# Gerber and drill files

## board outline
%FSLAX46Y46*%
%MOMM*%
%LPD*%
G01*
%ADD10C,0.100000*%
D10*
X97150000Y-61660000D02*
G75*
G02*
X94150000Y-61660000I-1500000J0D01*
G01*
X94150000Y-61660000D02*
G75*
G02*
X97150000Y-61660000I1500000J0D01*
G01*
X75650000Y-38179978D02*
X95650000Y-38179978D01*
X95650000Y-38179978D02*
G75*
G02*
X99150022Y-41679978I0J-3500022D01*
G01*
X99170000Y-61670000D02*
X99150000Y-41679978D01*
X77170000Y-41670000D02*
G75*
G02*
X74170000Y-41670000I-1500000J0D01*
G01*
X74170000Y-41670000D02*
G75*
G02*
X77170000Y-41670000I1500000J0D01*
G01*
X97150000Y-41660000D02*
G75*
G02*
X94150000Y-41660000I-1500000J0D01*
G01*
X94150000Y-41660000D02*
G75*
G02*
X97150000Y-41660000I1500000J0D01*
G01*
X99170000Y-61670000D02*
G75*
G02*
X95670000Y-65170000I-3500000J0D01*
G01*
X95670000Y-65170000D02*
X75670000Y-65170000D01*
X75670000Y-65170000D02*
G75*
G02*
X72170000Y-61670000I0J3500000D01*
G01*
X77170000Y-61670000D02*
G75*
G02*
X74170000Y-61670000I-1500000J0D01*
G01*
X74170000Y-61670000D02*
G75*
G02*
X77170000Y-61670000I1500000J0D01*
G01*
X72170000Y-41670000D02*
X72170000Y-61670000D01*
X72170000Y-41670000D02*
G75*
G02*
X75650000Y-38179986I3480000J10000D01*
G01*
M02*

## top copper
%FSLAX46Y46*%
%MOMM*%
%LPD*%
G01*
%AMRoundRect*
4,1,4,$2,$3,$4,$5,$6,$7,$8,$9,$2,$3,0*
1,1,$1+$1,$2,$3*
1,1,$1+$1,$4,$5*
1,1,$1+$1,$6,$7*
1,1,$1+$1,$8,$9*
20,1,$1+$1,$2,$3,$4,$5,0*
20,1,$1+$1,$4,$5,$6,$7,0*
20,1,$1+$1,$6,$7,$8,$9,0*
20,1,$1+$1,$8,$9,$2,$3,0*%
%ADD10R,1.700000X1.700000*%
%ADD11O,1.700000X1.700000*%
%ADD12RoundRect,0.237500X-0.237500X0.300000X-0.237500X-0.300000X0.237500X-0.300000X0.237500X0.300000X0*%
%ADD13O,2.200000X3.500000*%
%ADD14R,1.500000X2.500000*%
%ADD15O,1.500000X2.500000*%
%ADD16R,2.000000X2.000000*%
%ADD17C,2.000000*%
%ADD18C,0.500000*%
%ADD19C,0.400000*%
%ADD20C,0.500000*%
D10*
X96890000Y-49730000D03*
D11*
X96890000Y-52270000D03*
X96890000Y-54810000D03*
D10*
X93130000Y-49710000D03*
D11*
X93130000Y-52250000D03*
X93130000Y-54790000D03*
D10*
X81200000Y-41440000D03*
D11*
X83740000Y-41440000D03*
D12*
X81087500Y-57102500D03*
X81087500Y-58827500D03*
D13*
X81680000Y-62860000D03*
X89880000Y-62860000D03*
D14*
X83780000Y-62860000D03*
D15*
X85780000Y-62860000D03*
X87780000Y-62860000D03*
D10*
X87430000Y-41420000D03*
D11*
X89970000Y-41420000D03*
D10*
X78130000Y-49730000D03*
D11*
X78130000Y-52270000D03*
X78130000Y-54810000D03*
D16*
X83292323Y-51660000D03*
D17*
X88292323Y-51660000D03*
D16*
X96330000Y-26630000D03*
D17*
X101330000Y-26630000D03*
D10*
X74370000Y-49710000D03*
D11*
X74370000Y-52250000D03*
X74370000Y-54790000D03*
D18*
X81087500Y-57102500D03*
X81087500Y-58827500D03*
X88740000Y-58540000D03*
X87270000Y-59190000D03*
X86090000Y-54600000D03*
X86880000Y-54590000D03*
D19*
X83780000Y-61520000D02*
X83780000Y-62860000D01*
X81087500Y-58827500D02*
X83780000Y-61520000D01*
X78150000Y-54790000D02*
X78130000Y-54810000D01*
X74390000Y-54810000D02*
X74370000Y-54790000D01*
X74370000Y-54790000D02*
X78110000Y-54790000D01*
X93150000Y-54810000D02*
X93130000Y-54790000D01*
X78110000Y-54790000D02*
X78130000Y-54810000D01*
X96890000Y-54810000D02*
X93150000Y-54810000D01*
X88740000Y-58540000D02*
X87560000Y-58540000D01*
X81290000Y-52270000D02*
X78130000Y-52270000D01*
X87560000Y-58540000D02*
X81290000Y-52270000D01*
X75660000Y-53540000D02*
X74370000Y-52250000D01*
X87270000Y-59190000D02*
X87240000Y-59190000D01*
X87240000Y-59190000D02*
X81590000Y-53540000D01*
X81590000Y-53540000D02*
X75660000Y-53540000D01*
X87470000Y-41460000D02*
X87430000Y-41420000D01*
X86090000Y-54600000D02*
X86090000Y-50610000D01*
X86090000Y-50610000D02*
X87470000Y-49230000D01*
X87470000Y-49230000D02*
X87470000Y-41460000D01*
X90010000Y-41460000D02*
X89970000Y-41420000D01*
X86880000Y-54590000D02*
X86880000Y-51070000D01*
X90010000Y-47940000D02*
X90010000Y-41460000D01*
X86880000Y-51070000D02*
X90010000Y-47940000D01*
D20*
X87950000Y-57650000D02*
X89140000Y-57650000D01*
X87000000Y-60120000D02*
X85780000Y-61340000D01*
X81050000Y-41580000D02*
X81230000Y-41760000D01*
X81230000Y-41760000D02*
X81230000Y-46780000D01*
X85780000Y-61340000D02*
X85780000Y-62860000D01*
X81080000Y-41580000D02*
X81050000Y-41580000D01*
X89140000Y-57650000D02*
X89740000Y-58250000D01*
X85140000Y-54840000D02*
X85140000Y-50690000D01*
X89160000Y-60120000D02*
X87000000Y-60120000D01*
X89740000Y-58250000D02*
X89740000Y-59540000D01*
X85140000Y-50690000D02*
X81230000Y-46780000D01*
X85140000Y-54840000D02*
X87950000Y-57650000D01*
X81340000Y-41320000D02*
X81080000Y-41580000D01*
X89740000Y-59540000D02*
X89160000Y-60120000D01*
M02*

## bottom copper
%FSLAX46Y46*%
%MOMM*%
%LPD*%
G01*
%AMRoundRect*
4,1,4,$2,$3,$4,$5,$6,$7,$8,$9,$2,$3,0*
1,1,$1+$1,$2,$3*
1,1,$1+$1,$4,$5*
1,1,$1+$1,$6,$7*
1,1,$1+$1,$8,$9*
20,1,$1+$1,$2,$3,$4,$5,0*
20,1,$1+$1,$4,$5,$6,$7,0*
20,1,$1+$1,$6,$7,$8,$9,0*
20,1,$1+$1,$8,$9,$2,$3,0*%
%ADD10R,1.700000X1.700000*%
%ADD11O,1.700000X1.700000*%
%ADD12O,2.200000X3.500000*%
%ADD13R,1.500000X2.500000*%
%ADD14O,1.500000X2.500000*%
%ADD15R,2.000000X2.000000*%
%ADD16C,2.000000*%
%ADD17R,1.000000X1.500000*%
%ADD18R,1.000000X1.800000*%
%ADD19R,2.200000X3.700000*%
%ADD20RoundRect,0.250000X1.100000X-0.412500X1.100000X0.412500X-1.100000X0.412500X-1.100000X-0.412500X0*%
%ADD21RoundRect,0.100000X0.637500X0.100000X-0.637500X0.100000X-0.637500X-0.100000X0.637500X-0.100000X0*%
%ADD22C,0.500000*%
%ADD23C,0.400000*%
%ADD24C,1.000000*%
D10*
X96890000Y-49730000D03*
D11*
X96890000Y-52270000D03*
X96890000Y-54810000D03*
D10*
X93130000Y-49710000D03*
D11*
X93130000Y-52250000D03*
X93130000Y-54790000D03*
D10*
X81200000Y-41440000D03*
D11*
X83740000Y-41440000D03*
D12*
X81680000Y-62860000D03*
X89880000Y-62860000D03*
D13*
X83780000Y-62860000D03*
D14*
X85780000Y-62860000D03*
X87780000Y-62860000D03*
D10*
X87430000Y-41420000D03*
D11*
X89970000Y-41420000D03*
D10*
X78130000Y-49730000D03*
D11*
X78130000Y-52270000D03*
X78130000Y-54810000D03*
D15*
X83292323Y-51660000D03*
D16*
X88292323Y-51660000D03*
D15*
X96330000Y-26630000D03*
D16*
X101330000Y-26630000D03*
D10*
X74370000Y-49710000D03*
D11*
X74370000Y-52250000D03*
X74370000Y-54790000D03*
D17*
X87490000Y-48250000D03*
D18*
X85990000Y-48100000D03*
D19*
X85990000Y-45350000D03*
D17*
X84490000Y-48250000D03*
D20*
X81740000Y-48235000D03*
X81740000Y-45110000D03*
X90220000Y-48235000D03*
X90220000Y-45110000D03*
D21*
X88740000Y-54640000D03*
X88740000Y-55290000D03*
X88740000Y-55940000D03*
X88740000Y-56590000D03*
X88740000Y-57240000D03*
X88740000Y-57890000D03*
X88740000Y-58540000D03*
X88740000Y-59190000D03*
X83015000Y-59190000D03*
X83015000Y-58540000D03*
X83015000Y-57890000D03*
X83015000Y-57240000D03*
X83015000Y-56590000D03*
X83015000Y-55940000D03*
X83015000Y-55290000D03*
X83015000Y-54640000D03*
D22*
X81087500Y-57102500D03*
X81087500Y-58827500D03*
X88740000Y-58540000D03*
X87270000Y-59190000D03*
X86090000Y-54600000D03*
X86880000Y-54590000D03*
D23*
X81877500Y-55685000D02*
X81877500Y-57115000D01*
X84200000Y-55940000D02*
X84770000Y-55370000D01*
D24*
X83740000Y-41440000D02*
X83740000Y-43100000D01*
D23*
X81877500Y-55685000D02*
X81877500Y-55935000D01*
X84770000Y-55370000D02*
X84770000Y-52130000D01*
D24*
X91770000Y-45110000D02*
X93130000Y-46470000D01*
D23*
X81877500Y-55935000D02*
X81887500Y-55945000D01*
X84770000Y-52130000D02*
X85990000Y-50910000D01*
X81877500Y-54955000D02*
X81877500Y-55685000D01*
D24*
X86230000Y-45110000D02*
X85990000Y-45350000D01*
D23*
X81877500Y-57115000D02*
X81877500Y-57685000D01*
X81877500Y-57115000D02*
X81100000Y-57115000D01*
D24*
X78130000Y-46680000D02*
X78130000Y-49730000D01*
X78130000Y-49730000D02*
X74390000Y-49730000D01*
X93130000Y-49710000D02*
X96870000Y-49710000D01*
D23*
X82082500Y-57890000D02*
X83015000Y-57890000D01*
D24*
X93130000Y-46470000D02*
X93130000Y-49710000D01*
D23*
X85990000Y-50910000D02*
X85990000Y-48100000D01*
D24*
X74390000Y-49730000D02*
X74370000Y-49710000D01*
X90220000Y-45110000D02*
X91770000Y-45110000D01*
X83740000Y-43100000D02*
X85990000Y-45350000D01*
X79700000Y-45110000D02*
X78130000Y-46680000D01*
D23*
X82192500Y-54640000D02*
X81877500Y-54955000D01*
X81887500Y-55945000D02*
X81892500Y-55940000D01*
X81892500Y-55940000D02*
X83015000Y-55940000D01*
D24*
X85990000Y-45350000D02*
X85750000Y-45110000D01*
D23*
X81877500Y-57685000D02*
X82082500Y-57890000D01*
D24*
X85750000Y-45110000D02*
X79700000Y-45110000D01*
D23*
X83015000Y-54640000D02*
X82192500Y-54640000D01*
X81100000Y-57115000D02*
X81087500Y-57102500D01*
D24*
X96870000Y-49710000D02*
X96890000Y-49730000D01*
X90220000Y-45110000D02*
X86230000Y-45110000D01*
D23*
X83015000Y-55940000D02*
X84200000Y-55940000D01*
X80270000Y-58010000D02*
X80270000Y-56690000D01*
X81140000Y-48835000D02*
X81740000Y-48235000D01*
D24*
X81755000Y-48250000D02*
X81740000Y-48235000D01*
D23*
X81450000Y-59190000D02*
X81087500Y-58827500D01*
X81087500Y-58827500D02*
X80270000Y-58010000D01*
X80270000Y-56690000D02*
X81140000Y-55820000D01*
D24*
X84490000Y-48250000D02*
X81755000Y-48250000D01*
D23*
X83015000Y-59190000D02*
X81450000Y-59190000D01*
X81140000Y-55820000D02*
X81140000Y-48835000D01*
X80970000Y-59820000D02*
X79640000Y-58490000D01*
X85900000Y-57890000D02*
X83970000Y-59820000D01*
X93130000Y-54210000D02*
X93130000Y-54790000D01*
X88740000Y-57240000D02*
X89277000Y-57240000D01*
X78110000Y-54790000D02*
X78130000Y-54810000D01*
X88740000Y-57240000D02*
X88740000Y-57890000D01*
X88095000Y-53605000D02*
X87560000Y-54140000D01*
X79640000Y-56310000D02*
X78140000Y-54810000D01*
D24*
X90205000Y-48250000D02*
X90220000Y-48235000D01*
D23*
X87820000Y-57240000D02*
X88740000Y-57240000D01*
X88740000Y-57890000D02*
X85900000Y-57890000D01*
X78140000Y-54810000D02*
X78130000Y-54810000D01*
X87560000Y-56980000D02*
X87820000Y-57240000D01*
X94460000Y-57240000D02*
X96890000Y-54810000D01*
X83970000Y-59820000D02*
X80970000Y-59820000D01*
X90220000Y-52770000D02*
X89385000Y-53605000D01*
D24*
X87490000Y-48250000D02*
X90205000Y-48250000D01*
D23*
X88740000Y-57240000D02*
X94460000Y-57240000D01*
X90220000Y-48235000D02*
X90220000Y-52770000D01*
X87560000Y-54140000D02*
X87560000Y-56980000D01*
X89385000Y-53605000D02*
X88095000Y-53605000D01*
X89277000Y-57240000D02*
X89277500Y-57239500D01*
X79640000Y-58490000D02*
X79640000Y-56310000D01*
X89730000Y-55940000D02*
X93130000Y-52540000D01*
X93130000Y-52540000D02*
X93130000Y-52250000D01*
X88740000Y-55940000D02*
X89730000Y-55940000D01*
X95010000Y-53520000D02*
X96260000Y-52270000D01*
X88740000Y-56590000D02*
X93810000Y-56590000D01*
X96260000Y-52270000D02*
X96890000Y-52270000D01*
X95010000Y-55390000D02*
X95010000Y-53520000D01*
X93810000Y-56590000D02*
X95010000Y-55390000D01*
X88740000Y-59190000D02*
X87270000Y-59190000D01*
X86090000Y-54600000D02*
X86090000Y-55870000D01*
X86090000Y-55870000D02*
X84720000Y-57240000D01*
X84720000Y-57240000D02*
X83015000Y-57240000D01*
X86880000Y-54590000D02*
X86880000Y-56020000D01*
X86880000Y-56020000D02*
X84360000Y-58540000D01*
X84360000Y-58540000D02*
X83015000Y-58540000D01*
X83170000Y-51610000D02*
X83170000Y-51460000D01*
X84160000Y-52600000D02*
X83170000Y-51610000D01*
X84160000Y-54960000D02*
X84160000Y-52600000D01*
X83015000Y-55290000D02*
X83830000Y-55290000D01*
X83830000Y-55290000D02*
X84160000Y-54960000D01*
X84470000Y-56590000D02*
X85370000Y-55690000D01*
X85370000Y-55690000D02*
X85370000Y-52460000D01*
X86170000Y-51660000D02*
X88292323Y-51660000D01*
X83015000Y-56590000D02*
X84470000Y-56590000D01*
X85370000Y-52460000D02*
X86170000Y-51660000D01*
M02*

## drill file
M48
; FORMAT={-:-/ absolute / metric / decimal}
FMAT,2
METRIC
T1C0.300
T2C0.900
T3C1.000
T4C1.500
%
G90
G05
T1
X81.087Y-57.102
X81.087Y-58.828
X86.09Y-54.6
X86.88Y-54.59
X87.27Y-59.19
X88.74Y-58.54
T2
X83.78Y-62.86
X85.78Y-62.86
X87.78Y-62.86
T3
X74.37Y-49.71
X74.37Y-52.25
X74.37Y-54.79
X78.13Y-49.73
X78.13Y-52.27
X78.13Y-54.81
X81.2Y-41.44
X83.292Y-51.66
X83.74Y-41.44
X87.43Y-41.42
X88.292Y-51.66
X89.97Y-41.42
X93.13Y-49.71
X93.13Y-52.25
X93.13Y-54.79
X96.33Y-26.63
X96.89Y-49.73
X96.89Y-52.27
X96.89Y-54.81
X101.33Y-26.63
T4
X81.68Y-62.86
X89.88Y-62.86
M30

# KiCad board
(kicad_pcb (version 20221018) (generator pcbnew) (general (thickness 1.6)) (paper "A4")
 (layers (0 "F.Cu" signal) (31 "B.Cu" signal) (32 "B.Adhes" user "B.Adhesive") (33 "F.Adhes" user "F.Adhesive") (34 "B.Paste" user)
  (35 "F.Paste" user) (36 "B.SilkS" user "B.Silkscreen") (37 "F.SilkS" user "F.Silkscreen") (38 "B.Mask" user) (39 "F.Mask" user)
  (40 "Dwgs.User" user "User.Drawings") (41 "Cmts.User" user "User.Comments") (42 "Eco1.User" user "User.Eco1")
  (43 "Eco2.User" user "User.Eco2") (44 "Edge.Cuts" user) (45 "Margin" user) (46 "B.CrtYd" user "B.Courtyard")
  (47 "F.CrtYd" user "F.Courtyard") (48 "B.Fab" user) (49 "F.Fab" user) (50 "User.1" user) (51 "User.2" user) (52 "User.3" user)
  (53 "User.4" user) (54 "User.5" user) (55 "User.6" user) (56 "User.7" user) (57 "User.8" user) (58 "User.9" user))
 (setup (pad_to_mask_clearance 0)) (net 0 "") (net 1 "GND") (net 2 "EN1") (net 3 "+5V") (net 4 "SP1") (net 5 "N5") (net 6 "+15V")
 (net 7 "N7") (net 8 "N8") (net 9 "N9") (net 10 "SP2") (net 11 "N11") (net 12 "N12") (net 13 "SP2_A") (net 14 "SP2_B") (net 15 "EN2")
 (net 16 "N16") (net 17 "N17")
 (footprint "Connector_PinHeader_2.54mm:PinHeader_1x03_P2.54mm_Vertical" (layer "F.Cu") (at 96.89 49.73)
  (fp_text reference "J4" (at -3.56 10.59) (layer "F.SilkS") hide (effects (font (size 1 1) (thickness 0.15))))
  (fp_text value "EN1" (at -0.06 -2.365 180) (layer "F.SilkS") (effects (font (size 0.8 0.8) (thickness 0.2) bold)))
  (pad "1" thru_hole rect (at 0 0) (size 1.7 1.7) (drill 1) (layers "*.Cu" "*.Mask") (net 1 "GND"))
  (pad "2" thru_hole oval (at 0 2.54) (size 1.7 1.7) (drill 1) (layers "*.Cu" "*.Mask") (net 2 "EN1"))
  (pad "3" thru_hole oval (at 0 5.08) (size 1.7 1.7) (drill 1) (layers "*.Cu" "*.Mask") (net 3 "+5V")))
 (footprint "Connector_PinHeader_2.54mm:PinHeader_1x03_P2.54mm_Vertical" (layer "F.Cu") (at 93.13 49.71)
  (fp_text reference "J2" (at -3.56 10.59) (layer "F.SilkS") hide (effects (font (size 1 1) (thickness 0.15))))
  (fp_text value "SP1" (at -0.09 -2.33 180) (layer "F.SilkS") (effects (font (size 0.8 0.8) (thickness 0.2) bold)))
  (pad "1" thru_hole rect (at 0 0) (size 1.7 1.7) (drill 1) (layers "*.Cu" "*.Mask") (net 1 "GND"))
  (pad "2" thru_hole oval (at 0 2.54) (size 1.7 1.7) (drill 1) (layers "*.Cu" "*.Mask") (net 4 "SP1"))
  (pad "3" thru_hole oval (at 0 5.08) (size 1.7 1.7) (drill 1) (layers "*.Cu" "*.Mask") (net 3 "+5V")))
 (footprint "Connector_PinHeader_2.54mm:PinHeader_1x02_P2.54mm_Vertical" (layer "F.Cu") (at 81.2 41.44 90)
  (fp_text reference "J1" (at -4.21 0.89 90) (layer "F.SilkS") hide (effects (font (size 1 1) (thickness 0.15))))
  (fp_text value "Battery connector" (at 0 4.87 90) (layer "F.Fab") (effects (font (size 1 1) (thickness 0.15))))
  (pad "1" thru_hole rect (at 0 0 90) (size 1.7 1.7) (drill 1) (layers "*.Cu" "*.Mask") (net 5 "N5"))
  (pad "2" thru_hole oval (at 0 2.54 90) (size 1.7 1.7) (drill 1) (layers "*.Cu" "*.Mask") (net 1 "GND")))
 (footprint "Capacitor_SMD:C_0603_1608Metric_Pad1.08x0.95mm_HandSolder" (layer "F.Cu") (at 81.0875 57.965 -90)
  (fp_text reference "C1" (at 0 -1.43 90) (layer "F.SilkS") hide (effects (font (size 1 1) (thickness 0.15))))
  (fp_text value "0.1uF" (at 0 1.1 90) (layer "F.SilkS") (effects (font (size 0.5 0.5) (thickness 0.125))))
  (pad "1" smd roundrect (at -0.8625 0 270) (size 1.075 0.95) (layers "F.Cu" "F.Paste" "F.Mask") (roundrect_rratio 0.25) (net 1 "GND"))
  (pad "2" smd roundrect (at 0.8625 0 270) (size 1.075 0.95) (layers "F.Cu" "F.Paste" "F.Mask") (roundrect_rratio 0.25) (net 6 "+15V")))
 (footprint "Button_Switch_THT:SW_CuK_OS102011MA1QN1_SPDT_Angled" (layer "F.Cu") (at 83.78 62.86)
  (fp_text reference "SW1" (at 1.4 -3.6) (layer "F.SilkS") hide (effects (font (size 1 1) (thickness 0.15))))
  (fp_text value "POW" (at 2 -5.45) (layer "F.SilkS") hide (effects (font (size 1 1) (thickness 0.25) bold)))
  (pad "" thru_hole oval (at -2.1 0) (size 2.2 3.5) (drill 1.5) (layers "*.Cu" "*.Mask"))
  (pad "" thru_hole oval (at 6.1 0) (size 2.2 3.5) (drill 1.5) (layers "*.Cu" "*.Mask"))
  (pad "1" thru_hole rect (at 0 0) (size 1.5 2.5) (drill 0.9) (layers "*.Cu" "*.Mask") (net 6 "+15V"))
  (pad "2" thru_hole oval (at 2 0) (size 1.5 2.5) (drill 0.9) (layers "*.Cu" "*.Mask") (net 5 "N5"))
  (pad "3" thru_hole oval (at 4 0) (size 1.5 2.5) (drill 0.9) (layers "*.Cu" "*.Mask") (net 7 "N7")))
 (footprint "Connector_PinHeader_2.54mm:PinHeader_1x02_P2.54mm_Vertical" (layer "F.Cu") (at 87.43 41.42 90)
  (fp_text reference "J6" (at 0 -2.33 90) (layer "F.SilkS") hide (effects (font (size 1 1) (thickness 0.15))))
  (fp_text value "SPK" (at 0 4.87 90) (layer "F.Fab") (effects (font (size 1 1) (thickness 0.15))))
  (pad "1" thru_hole rect (at 0 0 90) (size 1.7 1.7) (drill 1) (layers "*.Cu" "*.Mask") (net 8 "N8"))
  (pad "2" thru_hole oval (at 0 2.54 90) (size 1.7 1.7) (drill 1) (layers "*.Cu" "*.Mask") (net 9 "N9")))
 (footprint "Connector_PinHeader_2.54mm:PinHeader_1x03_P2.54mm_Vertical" (layer "F.Cu") (at 78.13 49.73)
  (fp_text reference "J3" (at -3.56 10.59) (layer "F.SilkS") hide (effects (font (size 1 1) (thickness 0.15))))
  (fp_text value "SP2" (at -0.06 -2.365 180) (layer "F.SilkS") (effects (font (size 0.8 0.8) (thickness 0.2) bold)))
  (pad "1" thru_hole rect (at 0 0) (size 1.7 1.7) (drill 1) (layers "*.Cu" "*.Mask") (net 1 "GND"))
  (pad "2" thru_hole oval (at 0 2.54) (size 1.7 1.7) (drill 1) (layers "*.Cu" "*.Mask") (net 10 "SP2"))
  (pad "3" thru_hole oval (at 0 5.08) (size 1.7 1.7) (drill 1) (layers "*.Cu" "*.Mask") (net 3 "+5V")))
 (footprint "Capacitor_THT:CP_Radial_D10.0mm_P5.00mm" (layer "F.Cu") (at 83.292323 51.66)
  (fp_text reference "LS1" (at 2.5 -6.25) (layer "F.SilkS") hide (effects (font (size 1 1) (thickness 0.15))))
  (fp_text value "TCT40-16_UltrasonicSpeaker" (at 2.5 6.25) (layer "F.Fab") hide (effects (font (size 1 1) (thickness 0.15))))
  (pad "1" thru_hole rect (at 0 0) (size 2 2) (drill 1) (layers "*.Cu" "*.Mask") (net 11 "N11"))
  (pad "2" thru_hole circle (at 5 0) (size 2 2) (drill 1) (layers "*.Cu" "*.Mask") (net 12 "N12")))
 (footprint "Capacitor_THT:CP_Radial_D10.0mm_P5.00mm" (layer "F.Cu") (at 96.33 26.63)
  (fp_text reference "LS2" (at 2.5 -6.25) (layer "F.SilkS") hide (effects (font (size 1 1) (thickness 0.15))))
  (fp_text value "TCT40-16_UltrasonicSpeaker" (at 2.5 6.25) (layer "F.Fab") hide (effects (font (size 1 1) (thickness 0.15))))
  (pad "1" thru_hole rect (at 0 0) (size 2 2) (drill 1) (layers "*.Cu" "*.Mask") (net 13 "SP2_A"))
  (pad "2" thru_hole circle (at 5 0) (size 2 2) (drill 1) (layers "*.Cu" "*.Mask") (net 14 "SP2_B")))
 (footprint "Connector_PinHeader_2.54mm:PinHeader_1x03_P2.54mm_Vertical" (layer "F.Cu") (at 74.37 49.71)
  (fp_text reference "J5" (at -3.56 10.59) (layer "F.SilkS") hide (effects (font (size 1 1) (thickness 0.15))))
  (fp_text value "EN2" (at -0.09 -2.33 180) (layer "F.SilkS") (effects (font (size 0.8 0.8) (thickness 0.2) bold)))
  (pad "1" thru_hole rect (at 0 0) (size 1.7 1.7) (drill 1) (layers "*.Cu" "*.Mask") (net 1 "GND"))
  (pad "2" thru_hole oval (at 0 2.54) (size 1.7 1.7) (drill 1) (layers "*.Cu" "*.Mask") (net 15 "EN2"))
  (pad "3" thru_hole oval (at 0 5.08) (size 1.7 1.7) (drill 1) (layers "*.Cu" "*.Mask") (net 3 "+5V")))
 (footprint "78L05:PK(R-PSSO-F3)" (layer "B.Cu") (at 85.99 44.6 180)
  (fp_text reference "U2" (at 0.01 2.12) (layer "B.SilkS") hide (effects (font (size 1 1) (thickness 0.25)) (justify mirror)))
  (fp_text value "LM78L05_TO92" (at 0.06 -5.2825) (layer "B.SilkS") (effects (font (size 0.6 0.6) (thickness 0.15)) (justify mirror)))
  (pad "1" smd rect (at -1.5 -3.65 180) (size 1 1.5) (layers "B.Cu" "B.Paste" "B.Mask") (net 3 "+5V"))
  (pad "2" smd rect (at 0 -3.5 180) (size 1 1.8) (layers "B.Cu" "B.Paste" "B.Mask") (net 1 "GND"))
  (pad "2" smd rect (at 0 -0.75 180) (size 2.2 3.7) (layers "B.Cu" "B.Paste" "B.Mask") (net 1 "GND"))
  (pad "3" smd rect (at 1.5 -3.65 180) (size 1 1.5) (layers "B.Cu" "B.Paste" "B.Mask") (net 6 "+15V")))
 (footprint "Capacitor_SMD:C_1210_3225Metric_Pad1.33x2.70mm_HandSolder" (layer "B.Cu") (at 81.74 46.6725 90)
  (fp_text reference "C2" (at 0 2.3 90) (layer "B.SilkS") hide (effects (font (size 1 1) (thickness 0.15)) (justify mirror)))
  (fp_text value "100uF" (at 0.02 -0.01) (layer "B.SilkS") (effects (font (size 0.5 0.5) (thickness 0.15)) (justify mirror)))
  (pad "1" smd roundrect (at -1.5625 0 90) (size 1.325 2.7) (layers "B.Cu" "B.Paste" "B.Mask") (roundrect_rratio 0.188679) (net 6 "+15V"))
  (pad "2" smd roundrect (at 1.5625 0 90) (size 1.325 2.7) (layers "B.Cu" "B.Paste" "B.Mask") (roundrect_rratio 0.188679) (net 1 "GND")))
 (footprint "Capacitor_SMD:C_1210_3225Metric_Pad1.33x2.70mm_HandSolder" (layer "B.Cu") (at 90.22 46.6725 90)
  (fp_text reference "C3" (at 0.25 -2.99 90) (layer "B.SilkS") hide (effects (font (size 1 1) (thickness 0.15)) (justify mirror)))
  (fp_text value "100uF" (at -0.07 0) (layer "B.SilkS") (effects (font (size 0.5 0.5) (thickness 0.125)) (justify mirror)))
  (pad "1" smd roundrect (at -1.5625 0 90) (size 1.325 2.7) (layers "B.Cu" "B.Paste" "B.Mask") (roundrect_rratio 0.188679) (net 3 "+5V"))
  (pad "2" smd roundrect (at 1.5625 0 90) (size 1.325 2.7) (layers "B.Cu" "B.Paste" "B.Mask") (roundrect_rratio 0.188679) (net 1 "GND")))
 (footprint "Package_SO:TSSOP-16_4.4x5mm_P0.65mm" (layer "B.Cu") (at 85.8775 56.915 180)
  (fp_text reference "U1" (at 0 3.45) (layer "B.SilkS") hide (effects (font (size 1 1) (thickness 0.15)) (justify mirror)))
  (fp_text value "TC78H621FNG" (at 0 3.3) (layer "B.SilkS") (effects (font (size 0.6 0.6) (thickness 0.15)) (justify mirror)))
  (pad "1" smd roundrect (at -2.8625 2.275 180) (size 1.475 0.4) (layers "B.Cu" "B.Paste" "B.Mask") (roundrect_rratio 0.25) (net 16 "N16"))
  (pad "2" smd roundrect (at -2.8625 1.625 180) (size 1.475 0.4) (layers "B.Cu" "B.Paste" "B.Mask") (roundrect_rratio 0.25) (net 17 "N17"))
  (pad "3" smd roundrect (at -2.8625 0.975 180) (size 1.475 0.4) (layers "B.Cu" "B.Paste" "B.Mask") (roundrect_rratio 0.25) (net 4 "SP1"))
  (pad "4" smd roundrect (at -2.8625 0.325 180) (size 1.475 0.4) (layers "B.Cu" "B.Paste" "B.Mask") (roundrect_rratio 0.25) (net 2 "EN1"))
  (pad "5" smd roundrect (at -2.8625 -0.325 180) (size 1.475 0.4) (layers "B.Cu" "B.Paste" "B.Mask") (roundrect_rratio 0.25) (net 3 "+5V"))
  (pad "6" smd roundrect (at -2.8625 -0.975 180) (size 1.475 0.4) (layers "B.Cu" "B.Paste" "B.Mask") (roundrect_rratio 0.25) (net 3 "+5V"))
  (pad "7" smd roundrect (at -2.8625 -1.625 180) (size 1.475 0.4) (layers "B.Cu" "B.Paste" "B.Mask") (roundrect_rratio 0.25) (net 10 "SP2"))
  (pad "8" smd roundrect (at -2.8625 -2.275 180) (size 1.475 0.4) (layers "B.Cu" "B.Paste" "B.Mask") (roundrect_rratio 0.25) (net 15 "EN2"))
  (pad "9" smd roundrect (at 2.8625 -2.275 180) (size 1.475 0.4) (layers "B.Cu" "B.Paste" "B.Mask") (roundrect_rratio 0.25) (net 6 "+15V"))
  (pad "10" smd roundrect (at 2.8625 -1.625 180) (size 1.475 0.4) (layers "B.Cu" "B.Paste" "B.Mask") (roundrect_rratio 0.25) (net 9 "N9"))
  (pad "11" smd roundrect (at 2.8625 -0.975 180) (size 1.475 0.4) (layers "B.Cu" "B.Paste" "B.Mask") (roundrect_rratio 0.25) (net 1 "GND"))
  (pad "12" smd roundrect (at 2.8625 -0.325 180) (size 1.475 0.4) (layers "B.Cu" "B.Paste" "B.Mask") (roundrect_rratio 0.25) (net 8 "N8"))
  (pad "13" smd roundrect (at 2.8625 0.325 180) (size 1.475 0.4) (layers "B.Cu" "B.Paste" "B.Mask") (roundrect_rratio 0.25) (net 12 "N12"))
  (pad "14" smd roundrect (at 2.8625 0.975 180) (size 1.475 0.4) (layers "B.Cu" "B.Paste" "B.Mask") (roundrect_rratio 0.25) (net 1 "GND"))
  (pad "15" smd roundrect (at 2.8625 1.625 180) (size 1.475 0.4) (layers "B.Cu" "B.Paste" "B.Mask") (roundrect_rratio 0.25) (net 11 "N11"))
  (pad "16" smd roundrect (at 2.8625 2.275 180) (size 1.475 0.4) (layers "B.Cu" "B.Paste" "B.Mask") (roundrect_rratio 0.25) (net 1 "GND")))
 (gr_circle (center 95.65 61.66) (end 95.65 60.16) (stroke (width 0.1) (type solid)) (fill none) (layer "Edge.Cuts"))
 (gr_line (start 75.65 38.179978) (end 95.65 38.179978) (stroke (width 0.1) (type default)) (layer "Edge.Cuts"))
 (gr_arc (start 95.65 38.179978) (mid 98.124874 39.205104) (end 99.15 41.679978) (stroke (width 0.1) (type default)) (layer "Edge.Cuts"))
 (gr_line (start 99.17 61.67) (end 99.15 41.679978) (stroke (width 0.1) (type default)) (layer "Edge.Cuts"))
 (gr_circle (center 75.67 41.67) (end 75.67 43.17) (stroke (width 0.1) (type solid)) (fill none) (layer "Edge.Cuts"))
 (gr_circle (center 95.65 41.66) (end 95.65 40.16) (stroke (width 0.1) (type solid)) (fill none) (layer "Edge.Cuts"))
 (gr_arc (start 99.17 61.67) (mid 98.144874 64.144874) (end 95.67 65.17) (stroke (width 0.1) (type default)) (layer "Edge.Cuts"))
 (gr_line (start 95.67 65.17) (end 75.67 65.17) (stroke (width 0.1) (type default)) (layer "Edge.Cuts"))
 (gr_arc (start 75.67 65.17) (mid 73.195126 64.144874) (end 72.17 61.67) (stroke (width 0.1) (type default)) (layer "Edge.Cuts"))
 (gr_circle (center 75.67 61.67) (end 75.67 63.17) (stroke (width 0.1) (type solid)) (fill none) (layer "Edge.Cuts"))
 (gr_line (start 72.17 41.67) (end 72.17 61.67) (stroke (width 0.1) (type default)) (layer "Edge.Cuts"))
 (gr_arc (start 72.17 41.67) (mid 73.185724 39.202792) (end 75.65 38.179978) (stroke (width 0.1) (type default)) (layer "Edge.Cuts"))
 (via (at 81.0875 57.1025) (size 0.5) (drill 0.3) (layers "F.Cu" "B.Cu") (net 1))
 (segment (start 81.8775 55.685) (end 81.8775 57.115) (width 0.4) (layer "B.Cu") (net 1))
 (segment (start 84.2 55.94) (end 84.77 55.37) (width 0.4) (layer "B.Cu") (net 1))
 (segment (start 83.74 41.44) (end 83.74 43.1) (width 1) (layer "B.Cu") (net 1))
 (segment (start 81.8775 55.685) (end 81.8775 55.935) (width 0.4) (layer "B.Cu") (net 1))
 (segment (start 84.77 55.37) (end 84.77 52.13) (width 0.4) (layer "B.Cu") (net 1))
 (segment (start 91.77 45.11) (end 93.13 46.47) (width 1) (layer "B.Cu") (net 1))
 (segment (start 81.8775 55.935) (end 81.8875 55.945) (width 0.4) (layer "B.Cu") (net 1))
 (segment (start 84.77 52.13) (end 85.99 50.91) (width 0.4) (layer "B.Cu") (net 1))
 (segment (start 81.8775 54.955) (end 81.8775 55.685) (width 0.4) (layer "B.Cu") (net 1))
 (segment (start 86.23 45.11) (end 85.99 45.35) (width 1) (layer "B.Cu") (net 1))
 (segment (start 81.8775 57.115) (end 81.8775 57.685) (width 0.4) (layer "B.Cu") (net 1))
 (segment (start 81.8775 57.115) (end 81.1 57.115) (width 0.4) (layer "B.Cu") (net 1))
 (segment (start 78.13 46.68) (end 78.13 49.73) (width 1) (layer "B.Cu") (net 1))
 (segment (start 78.13 49.73) (end 74.39 49.73) (width 1) (layer "B.Cu") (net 1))
 (segment (start 93.13 49.71) (end 96.87 49.71) (width 1) (layer "B.Cu") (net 1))
 (segment (start 82.0825 57.89) (end 83.015 57.89) (width 0.4) (layer "B.Cu") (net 1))
 (segment (start 93.13 46.47) (end 93.13 49.71) (width 1) (layer "B.Cu") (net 1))
 (segment (start 85.99 50.91) (end 85.99 48.1) (width 0.4) (layer "B.Cu") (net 1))
 (segment (start 74.39 49.73) (end 74.37 49.71) (width 1) (layer "B.Cu") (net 1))
 (segment (start 90.22 45.11) (end 91.77 45.11) (width 1) (layer "B.Cu") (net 1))
 (segment (start 83.74 43.1) (end 85.99 45.35) (width 1) (layer "B.Cu") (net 1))
 (segment (start 79.7 45.11) (end 78.13 46.68) (width 1) (layer "B.Cu") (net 1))
 (segment (start 82.1925 54.64) (end 81.8775 54.955) (width 0.4) (layer "B.Cu") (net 1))
 (segment (start 81.8875 55.945) (end 81.8925 55.94) (width 0.4) (layer "B.Cu") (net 1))
 (segment (start 81.8925 55.94) (end 83.015 55.94) (width 0.4) (layer "B.Cu") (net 1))
 (segment (start 85.99 45.35) (end 85.75 45.11) (width 1) (layer "B.Cu") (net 1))
 (segment (start 81.8775 57.685) (end 82.0825 57.89) (width 0.4) (layer "B.Cu") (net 1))
 (segment (start 85.75 45.11) (end 79.7 45.11) (width 1) (layer "B.Cu") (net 1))
 (segment (start 83.015 54.64) (end 82.1925 54.64) (width 0.4) (layer "B.Cu") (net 1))
 (segment (start 81.1 57.115) (end 81.0875 57.1025) (width 0.4) (layer "B.Cu") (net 1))
 (segment (start 96.87 49.71) (end 96.89 49.73) (width 1) (layer "B.Cu") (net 1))
 (segment (start 90.22 45.11) (end 86.23 45.11) (width 1) (layer "B.Cu") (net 1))
 (segment (start 83.015 55.94) (end 84.2 55.94) (width 0.4) (layer "B.Cu") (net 1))
 (segment (start 83.78 61.52) (end 83.78 62.86) (width 0.4) (layer "F.Cu") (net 6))
 (segment (start 81.0875 58.8275) (end 83.78 61.52) (width 0.4) (layer "F.Cu") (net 6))
 (via (at 81.0875 58.8275) (size 0.5) (drill 0.3) (layers "F.Cu" "B.Cu") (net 6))
 (segment (start 80.27 58.01) (end 80.27 56.69) (width 0.4) (layer "B.Cu") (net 6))
 (segment (start 81.14 48.835) (end 81.74 48.235) (width 0.4) (layer "B.Cu") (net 6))
 (segment (start 81.755 48.25) (end 81.74 48.235) (width 1) (layer "B.Cu") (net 6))
 (segment (start 81.45 59.19) (end 81.0875 58.8275) (width 0.4) (layer "B.Cu") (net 6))
 (segment (start 81.0875 58.8275) (end 80.27 58.01) (width 0.4) (layer "B.Cu") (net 6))
 (segment (start 80.27 56.69) (end 81.14 55.82) (width 0.4) (layer "B.Cu") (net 6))
 (segment (start 84.49 48.25) (end 81.755 48.25) (width 1) (layer "B.Cu") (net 6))
 (segment (start 83.015 59.19) (end 81.45 59.19) (width 0.4) (layer "B.Cu") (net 6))
 (segment (start 81.14 55.82) (end 81.14 48.835) (width 0.4) (layer "B.Cu") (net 6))
 (segment (start 78.15 54.79) (end 78.13 54.81) (width 0.4) (layer "F.Cu") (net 3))
 (segment (start 74.39 54.81) (end 74.37 54.79) (width 0.4) (layer "F.Cu") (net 3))
 (segment (start 74.37 54.79) (end 78.11 54.79) (width 0.4) (layer "F.Cu") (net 3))
 (segment (start 93.15 54.81) (end 93.13 54.79) (width 0.4) (layer "F.Cu") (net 3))
 (segment (start 78.11 54.79) (end 78.13 54.81) (width 0.4) (layer "F.Cu") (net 3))
 (segment (start 96.89 54.81) (end 93.15 54.81) (width 0.4) (layer "F.Cu") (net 3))
 (segment (start 80.97 59.82) (end 79.64 58.49) (width 0.4) (layer "B.Cu") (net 3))
 (segment (start 85.9 57.89) (end 83.97 59.82) (width 0.4) (layer "B.Cu") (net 3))
 (segment (start 93.13 54.21) (end 93.13 54.79) (width 0.4) (layer "B.Cu") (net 3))
 (segment (start 88.74 57.24) (end 89.277 57.24) (width 0.4) (layer "B.Cu") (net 3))
 (segment (start 78.11 54.79) (end 78.13 54.81) (width 0.4) (layer "B.Cu") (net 3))
 (segment (start 88.74 57.24) (end 88.74 57.89) (width 0.4) (layer "B.Cu") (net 3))
 (segment (start 88.095 53.605) (end 87.56 54.14) (width 0.4) (layer "B.Cu") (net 3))
 (segment (start 79.64 56.31) (end 78.14 54.81) (width 0.4) (layer "B.Cu") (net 3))
 (segment (start 90.205 48.25) (end 90.22 48.235) (width 1) (layer "B.Cu") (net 3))
 (segment (start 87.82 57.24) (end 88.74 57.24) (width 0.4) (layer "B.Cu") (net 3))
 (segment (start 88.74 57.89) (end 85.9 57.89) (width 0.4) (layer "B.Cu") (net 3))
 (segment (start 78.14 54.81) (end 78.13 54.81) (width 0.4) (layer "B.Cu") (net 3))
 (segment (start 87.56 56.98) (end 87.82 57.24) (width 0.4) (layer "B.Cu") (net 3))
 (segment (start 94.46 57.24) (end 96.89 54.81) (width 0.4) (layer "B.Cu") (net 3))
 (segment (start 83.97 59.82) (end 80.97 59.82) (width 0.4) (layer "B.Cu") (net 3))
 (segment (start 90.22 52.77) (end 89.385 53.605) (width 0.4) (layer "B.Cu") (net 3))
 (segment (start 87.49 48.25) (end 90.205 48.25) (width 1) (layer "B.Cu") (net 3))
 (segment (start 88.74 57.24) (end 94.46 57.24) (width 0.4) (layer "B.Cu") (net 3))
 (segment (start 90.22 48.235) (end 90.22 52.77) (width 0.4) (layer "B.Cu") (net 3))
 (segment (start 87.56 54.14) (end 87.56 56.98) (width 0.4) (layer "B.Cu") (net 3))
 (segment (start 89.385 53.605) (end 88.095 53.605) (width 0.4) (layer "B.Cu") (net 3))
 (segment (start 89.277 57.24) (end 89.2775 57.2395) (width 0.4) (layer "B.Cu") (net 3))
 (segment (start 79.64 58.49) (end 79.64 56.31) (width 0.4) (layer "B.Cu") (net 3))
 (segment (start 89.73 55.94) (end 93.13 52.54) (width 0.4) (layer "B.Cu") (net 4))
 (segment (start 93.13 52.54) (end 93.13 52.25) (width 0.4) (layer "B.Cu") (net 4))
 (segment (start 88.74 55.94) (end 89.73 55.94) (width 0.4) (layer "B.Cu") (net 4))
 (segment (start 88.74 58.54) (end 87.56 58.54) (width 0.4) (layer "F.Cu") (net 10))
 (segment (start 81.29 52.27) (end 78.13 52.27) (width 0.4) (layer "F.Cu") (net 10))
 (segment (start 87.56 58.54) (end 81.29 52.27) (width 0.4) (layer "F.Cu") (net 10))
 (via (at 88.74 58.54) (size 0.5) (drill 0.3) (layers "F.Cu" "B.Cu") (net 10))
 (segment (start 95.01 53.52) (end 96.26 52.27) (width 0.4) (layer "B.Cu") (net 2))
 (segment (start 88.74 56.59) (end 93.81 56.59) (width 0.4) (layer "B.Cu") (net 2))
 (segment (start 96.26 52.27) (end 96.89 52.27) (width 0.4) (layer "B.Cu") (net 2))
 (segment (start 95.01 55.39) (end 95.01 53.52) (width 0.4) (layer "B.Cu") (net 2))
 (segment (start 93.81 56.59) (end 95.01 55.39) (width 0.4) (layer "B.Cu") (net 2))
 (segment (start 75.66 53.54) (end 74.37 52.25) (width 0.4) (layer "F.Cu") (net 15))
 (segment (start 87.27 59.19) (end 87.24 59.19) (width 0.4) (layer "F.Cu") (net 15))
 (segment (start 87.24 59.19) (end 81.59 53.54) (width 0.4) (layer "F.Cu") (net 15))
 (segment (start 81.59 53.54) (end 75.66 53.54) (width 0.4) (layer "F.Cu") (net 15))
 (via (at 87.27 59.19) (size 0.5) (drill 0.3) (layers "F.Cu" "B.Cu") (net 15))
 (segment (start 88.74 59.19) (end 87.27 59.19) (width 0.4) (layer "B.Cu") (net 15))
 (segment (start 87.47 41.46) (end 87.43 41.42) (width 0.4) (layer "F.Cu") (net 8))
 (segment (start 86.09 54.6) (end 86.09 50.61) (width 0.4) (layer "F.Cu") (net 8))
 (segment (start 86.09 50.61) (end 87.47 49.23) (width 0.4) (layer "F.Cu") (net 8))
 (segment (start 87.47 49.23) (end 87.47 41.46) (width 0.4) (layer "F.Cu") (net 8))
 (via (at 86.09 54.6) (size 0.5) (drill 0.3) (layers "F.Cu" "B.Cu") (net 8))
 (segment (start 86.09 54.6) (end 86.09 55.87) (width 0.4) (layer "B.Cu") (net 8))
 (segment (start 86.09 55.87) (end 84.72 57.24) (width 0.4) (layer "B.Cu") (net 8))
 (segment (start 84.72 57.24) (end 83.015 57.24) (width 0.4) (layer "B.Cu") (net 8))
 (segment (start 90.01 41.46) (end 89.97 41.42) (width 0.4) (layer "F.Cu") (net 9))
 (segment (start 86.88 54.59) (end 86.88 51.07) (width 0.4) (layer "F.Cu") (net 9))
 (segment (start 90.01 47.94) (end 90.01 41.46) (width 0.4) (layer "F.Cu") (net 9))
 (segment (start 86.88 51.07) (end 90.01 47.94) (width 0.4) (layer "F.Cu") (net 9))
 (via (at 86.88 54.59) (size 0.5) (drill 0.3) (layers "F.Cu" "B.Cu") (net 9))
 (segment (start 86.88 54.59) (end 86.88 56.02) (width 0.4) (layer "B.Cu") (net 9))
 (segment (start 86.88 56.02) (end 84.36 58.54) (width 0.4) (layer "B.Cu") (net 9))
 (segment (start 84.36 58.54) (end 83.015 58.54) (width 0.4) (layer "B.Cu") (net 9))
 (segment (start 83.17 51.61) (end 83.17 51.46) (width 0.4) (layer "B.Cu") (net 11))
 (segment (start 84.16 52.6) (end 83.17 51.61) (width 0.4) (layer "B.Cu") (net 11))
 (segment (start 84.16 54.96) (end 84.16 52.6) (width 0.4) (layer "B.Cu") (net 11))
 (segment (start 83.015 55.29) (end 83.83 55.29) (width 0.4) (layer "B.Cu") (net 11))
 (segment (start 83.83 55.29) (end 84.16 54.96) (width 0.4) (layer "B.Cu") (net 11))
 (segment (start 84.47 56.59) (end 85.37 55.69) (width 0.4) (layer "B.Cu") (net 12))
 (segment (start 85.37 55.69) (end 85.37 52.46) (width 0.4) (layer "B.Cu") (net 12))
 (segment (start 86.17 51.66) (end 88.292323 51.66) (width 0.4) (layer "B.Cu") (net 12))
 (segment (start 83.015 56.59) (end 84.47 56.59) (width 0.4) (layer "B.Cu") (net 12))
 (segment (start 85.37 52.46) (end 86.17 51.66) (width 0.4) (layer "B.Cu") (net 12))
 (segment (start 87.95 57.65) (end 89.14 57.65) (width 0.5) (layer "F.Cu") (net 5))
 (segment (start 87 60.12) (end 85.78 61.34) (width 0.5) (layer "F.Cu") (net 5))
 (segment (start 81.05 41.58) (end 81.23 41.76) (width 0.5) (layer "F.Cu") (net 5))
 (segment (start 81.23 41.76) (end 81.23 46.78) (width 0.5) (layer "F.Cu") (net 5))
 (segment (start 85.78 61.34) (end 85.78 62.86) (width 0.5) (layer "F.Cu") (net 5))
 (segment (start 81.08 41.58) (end 81.05 41.58) (width 0.5) (layer "F.Cu") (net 5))
 (segment (start 89.14 57.65) (end 89.74 58.25) (width 0.5) (layer "F.Cu") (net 5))
 (segment (start 85.14 54.84) (end 85.14 50.69) (width 0.5) (layer "F.Cu") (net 5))
 (segment (start 89.16 60.12) (end 87 60.12) (width 0.5) (layer "F.Cu") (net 5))
 (segment (start 89.74 58.25) (end 89.74 59.54) (width 0.5) (layer "F.Cu") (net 5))
 (segment (start 85.14 50.69) (end 81.23 46.78) (width 0.5) (layer "F.Cu") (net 5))
 (segment (start 85.14 54.84) (end 87.95 57.65) (width 0.5) (layer "F.Cu") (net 5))
 (segment (start 81.34 41.32) (end 81.08 41.58) (width 0.5) (layer "F.Cu") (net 5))
 (segment (start 89.74 59.54) (end 89.16 60.12) (width 0.5) (layer "F.Cu") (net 5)))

